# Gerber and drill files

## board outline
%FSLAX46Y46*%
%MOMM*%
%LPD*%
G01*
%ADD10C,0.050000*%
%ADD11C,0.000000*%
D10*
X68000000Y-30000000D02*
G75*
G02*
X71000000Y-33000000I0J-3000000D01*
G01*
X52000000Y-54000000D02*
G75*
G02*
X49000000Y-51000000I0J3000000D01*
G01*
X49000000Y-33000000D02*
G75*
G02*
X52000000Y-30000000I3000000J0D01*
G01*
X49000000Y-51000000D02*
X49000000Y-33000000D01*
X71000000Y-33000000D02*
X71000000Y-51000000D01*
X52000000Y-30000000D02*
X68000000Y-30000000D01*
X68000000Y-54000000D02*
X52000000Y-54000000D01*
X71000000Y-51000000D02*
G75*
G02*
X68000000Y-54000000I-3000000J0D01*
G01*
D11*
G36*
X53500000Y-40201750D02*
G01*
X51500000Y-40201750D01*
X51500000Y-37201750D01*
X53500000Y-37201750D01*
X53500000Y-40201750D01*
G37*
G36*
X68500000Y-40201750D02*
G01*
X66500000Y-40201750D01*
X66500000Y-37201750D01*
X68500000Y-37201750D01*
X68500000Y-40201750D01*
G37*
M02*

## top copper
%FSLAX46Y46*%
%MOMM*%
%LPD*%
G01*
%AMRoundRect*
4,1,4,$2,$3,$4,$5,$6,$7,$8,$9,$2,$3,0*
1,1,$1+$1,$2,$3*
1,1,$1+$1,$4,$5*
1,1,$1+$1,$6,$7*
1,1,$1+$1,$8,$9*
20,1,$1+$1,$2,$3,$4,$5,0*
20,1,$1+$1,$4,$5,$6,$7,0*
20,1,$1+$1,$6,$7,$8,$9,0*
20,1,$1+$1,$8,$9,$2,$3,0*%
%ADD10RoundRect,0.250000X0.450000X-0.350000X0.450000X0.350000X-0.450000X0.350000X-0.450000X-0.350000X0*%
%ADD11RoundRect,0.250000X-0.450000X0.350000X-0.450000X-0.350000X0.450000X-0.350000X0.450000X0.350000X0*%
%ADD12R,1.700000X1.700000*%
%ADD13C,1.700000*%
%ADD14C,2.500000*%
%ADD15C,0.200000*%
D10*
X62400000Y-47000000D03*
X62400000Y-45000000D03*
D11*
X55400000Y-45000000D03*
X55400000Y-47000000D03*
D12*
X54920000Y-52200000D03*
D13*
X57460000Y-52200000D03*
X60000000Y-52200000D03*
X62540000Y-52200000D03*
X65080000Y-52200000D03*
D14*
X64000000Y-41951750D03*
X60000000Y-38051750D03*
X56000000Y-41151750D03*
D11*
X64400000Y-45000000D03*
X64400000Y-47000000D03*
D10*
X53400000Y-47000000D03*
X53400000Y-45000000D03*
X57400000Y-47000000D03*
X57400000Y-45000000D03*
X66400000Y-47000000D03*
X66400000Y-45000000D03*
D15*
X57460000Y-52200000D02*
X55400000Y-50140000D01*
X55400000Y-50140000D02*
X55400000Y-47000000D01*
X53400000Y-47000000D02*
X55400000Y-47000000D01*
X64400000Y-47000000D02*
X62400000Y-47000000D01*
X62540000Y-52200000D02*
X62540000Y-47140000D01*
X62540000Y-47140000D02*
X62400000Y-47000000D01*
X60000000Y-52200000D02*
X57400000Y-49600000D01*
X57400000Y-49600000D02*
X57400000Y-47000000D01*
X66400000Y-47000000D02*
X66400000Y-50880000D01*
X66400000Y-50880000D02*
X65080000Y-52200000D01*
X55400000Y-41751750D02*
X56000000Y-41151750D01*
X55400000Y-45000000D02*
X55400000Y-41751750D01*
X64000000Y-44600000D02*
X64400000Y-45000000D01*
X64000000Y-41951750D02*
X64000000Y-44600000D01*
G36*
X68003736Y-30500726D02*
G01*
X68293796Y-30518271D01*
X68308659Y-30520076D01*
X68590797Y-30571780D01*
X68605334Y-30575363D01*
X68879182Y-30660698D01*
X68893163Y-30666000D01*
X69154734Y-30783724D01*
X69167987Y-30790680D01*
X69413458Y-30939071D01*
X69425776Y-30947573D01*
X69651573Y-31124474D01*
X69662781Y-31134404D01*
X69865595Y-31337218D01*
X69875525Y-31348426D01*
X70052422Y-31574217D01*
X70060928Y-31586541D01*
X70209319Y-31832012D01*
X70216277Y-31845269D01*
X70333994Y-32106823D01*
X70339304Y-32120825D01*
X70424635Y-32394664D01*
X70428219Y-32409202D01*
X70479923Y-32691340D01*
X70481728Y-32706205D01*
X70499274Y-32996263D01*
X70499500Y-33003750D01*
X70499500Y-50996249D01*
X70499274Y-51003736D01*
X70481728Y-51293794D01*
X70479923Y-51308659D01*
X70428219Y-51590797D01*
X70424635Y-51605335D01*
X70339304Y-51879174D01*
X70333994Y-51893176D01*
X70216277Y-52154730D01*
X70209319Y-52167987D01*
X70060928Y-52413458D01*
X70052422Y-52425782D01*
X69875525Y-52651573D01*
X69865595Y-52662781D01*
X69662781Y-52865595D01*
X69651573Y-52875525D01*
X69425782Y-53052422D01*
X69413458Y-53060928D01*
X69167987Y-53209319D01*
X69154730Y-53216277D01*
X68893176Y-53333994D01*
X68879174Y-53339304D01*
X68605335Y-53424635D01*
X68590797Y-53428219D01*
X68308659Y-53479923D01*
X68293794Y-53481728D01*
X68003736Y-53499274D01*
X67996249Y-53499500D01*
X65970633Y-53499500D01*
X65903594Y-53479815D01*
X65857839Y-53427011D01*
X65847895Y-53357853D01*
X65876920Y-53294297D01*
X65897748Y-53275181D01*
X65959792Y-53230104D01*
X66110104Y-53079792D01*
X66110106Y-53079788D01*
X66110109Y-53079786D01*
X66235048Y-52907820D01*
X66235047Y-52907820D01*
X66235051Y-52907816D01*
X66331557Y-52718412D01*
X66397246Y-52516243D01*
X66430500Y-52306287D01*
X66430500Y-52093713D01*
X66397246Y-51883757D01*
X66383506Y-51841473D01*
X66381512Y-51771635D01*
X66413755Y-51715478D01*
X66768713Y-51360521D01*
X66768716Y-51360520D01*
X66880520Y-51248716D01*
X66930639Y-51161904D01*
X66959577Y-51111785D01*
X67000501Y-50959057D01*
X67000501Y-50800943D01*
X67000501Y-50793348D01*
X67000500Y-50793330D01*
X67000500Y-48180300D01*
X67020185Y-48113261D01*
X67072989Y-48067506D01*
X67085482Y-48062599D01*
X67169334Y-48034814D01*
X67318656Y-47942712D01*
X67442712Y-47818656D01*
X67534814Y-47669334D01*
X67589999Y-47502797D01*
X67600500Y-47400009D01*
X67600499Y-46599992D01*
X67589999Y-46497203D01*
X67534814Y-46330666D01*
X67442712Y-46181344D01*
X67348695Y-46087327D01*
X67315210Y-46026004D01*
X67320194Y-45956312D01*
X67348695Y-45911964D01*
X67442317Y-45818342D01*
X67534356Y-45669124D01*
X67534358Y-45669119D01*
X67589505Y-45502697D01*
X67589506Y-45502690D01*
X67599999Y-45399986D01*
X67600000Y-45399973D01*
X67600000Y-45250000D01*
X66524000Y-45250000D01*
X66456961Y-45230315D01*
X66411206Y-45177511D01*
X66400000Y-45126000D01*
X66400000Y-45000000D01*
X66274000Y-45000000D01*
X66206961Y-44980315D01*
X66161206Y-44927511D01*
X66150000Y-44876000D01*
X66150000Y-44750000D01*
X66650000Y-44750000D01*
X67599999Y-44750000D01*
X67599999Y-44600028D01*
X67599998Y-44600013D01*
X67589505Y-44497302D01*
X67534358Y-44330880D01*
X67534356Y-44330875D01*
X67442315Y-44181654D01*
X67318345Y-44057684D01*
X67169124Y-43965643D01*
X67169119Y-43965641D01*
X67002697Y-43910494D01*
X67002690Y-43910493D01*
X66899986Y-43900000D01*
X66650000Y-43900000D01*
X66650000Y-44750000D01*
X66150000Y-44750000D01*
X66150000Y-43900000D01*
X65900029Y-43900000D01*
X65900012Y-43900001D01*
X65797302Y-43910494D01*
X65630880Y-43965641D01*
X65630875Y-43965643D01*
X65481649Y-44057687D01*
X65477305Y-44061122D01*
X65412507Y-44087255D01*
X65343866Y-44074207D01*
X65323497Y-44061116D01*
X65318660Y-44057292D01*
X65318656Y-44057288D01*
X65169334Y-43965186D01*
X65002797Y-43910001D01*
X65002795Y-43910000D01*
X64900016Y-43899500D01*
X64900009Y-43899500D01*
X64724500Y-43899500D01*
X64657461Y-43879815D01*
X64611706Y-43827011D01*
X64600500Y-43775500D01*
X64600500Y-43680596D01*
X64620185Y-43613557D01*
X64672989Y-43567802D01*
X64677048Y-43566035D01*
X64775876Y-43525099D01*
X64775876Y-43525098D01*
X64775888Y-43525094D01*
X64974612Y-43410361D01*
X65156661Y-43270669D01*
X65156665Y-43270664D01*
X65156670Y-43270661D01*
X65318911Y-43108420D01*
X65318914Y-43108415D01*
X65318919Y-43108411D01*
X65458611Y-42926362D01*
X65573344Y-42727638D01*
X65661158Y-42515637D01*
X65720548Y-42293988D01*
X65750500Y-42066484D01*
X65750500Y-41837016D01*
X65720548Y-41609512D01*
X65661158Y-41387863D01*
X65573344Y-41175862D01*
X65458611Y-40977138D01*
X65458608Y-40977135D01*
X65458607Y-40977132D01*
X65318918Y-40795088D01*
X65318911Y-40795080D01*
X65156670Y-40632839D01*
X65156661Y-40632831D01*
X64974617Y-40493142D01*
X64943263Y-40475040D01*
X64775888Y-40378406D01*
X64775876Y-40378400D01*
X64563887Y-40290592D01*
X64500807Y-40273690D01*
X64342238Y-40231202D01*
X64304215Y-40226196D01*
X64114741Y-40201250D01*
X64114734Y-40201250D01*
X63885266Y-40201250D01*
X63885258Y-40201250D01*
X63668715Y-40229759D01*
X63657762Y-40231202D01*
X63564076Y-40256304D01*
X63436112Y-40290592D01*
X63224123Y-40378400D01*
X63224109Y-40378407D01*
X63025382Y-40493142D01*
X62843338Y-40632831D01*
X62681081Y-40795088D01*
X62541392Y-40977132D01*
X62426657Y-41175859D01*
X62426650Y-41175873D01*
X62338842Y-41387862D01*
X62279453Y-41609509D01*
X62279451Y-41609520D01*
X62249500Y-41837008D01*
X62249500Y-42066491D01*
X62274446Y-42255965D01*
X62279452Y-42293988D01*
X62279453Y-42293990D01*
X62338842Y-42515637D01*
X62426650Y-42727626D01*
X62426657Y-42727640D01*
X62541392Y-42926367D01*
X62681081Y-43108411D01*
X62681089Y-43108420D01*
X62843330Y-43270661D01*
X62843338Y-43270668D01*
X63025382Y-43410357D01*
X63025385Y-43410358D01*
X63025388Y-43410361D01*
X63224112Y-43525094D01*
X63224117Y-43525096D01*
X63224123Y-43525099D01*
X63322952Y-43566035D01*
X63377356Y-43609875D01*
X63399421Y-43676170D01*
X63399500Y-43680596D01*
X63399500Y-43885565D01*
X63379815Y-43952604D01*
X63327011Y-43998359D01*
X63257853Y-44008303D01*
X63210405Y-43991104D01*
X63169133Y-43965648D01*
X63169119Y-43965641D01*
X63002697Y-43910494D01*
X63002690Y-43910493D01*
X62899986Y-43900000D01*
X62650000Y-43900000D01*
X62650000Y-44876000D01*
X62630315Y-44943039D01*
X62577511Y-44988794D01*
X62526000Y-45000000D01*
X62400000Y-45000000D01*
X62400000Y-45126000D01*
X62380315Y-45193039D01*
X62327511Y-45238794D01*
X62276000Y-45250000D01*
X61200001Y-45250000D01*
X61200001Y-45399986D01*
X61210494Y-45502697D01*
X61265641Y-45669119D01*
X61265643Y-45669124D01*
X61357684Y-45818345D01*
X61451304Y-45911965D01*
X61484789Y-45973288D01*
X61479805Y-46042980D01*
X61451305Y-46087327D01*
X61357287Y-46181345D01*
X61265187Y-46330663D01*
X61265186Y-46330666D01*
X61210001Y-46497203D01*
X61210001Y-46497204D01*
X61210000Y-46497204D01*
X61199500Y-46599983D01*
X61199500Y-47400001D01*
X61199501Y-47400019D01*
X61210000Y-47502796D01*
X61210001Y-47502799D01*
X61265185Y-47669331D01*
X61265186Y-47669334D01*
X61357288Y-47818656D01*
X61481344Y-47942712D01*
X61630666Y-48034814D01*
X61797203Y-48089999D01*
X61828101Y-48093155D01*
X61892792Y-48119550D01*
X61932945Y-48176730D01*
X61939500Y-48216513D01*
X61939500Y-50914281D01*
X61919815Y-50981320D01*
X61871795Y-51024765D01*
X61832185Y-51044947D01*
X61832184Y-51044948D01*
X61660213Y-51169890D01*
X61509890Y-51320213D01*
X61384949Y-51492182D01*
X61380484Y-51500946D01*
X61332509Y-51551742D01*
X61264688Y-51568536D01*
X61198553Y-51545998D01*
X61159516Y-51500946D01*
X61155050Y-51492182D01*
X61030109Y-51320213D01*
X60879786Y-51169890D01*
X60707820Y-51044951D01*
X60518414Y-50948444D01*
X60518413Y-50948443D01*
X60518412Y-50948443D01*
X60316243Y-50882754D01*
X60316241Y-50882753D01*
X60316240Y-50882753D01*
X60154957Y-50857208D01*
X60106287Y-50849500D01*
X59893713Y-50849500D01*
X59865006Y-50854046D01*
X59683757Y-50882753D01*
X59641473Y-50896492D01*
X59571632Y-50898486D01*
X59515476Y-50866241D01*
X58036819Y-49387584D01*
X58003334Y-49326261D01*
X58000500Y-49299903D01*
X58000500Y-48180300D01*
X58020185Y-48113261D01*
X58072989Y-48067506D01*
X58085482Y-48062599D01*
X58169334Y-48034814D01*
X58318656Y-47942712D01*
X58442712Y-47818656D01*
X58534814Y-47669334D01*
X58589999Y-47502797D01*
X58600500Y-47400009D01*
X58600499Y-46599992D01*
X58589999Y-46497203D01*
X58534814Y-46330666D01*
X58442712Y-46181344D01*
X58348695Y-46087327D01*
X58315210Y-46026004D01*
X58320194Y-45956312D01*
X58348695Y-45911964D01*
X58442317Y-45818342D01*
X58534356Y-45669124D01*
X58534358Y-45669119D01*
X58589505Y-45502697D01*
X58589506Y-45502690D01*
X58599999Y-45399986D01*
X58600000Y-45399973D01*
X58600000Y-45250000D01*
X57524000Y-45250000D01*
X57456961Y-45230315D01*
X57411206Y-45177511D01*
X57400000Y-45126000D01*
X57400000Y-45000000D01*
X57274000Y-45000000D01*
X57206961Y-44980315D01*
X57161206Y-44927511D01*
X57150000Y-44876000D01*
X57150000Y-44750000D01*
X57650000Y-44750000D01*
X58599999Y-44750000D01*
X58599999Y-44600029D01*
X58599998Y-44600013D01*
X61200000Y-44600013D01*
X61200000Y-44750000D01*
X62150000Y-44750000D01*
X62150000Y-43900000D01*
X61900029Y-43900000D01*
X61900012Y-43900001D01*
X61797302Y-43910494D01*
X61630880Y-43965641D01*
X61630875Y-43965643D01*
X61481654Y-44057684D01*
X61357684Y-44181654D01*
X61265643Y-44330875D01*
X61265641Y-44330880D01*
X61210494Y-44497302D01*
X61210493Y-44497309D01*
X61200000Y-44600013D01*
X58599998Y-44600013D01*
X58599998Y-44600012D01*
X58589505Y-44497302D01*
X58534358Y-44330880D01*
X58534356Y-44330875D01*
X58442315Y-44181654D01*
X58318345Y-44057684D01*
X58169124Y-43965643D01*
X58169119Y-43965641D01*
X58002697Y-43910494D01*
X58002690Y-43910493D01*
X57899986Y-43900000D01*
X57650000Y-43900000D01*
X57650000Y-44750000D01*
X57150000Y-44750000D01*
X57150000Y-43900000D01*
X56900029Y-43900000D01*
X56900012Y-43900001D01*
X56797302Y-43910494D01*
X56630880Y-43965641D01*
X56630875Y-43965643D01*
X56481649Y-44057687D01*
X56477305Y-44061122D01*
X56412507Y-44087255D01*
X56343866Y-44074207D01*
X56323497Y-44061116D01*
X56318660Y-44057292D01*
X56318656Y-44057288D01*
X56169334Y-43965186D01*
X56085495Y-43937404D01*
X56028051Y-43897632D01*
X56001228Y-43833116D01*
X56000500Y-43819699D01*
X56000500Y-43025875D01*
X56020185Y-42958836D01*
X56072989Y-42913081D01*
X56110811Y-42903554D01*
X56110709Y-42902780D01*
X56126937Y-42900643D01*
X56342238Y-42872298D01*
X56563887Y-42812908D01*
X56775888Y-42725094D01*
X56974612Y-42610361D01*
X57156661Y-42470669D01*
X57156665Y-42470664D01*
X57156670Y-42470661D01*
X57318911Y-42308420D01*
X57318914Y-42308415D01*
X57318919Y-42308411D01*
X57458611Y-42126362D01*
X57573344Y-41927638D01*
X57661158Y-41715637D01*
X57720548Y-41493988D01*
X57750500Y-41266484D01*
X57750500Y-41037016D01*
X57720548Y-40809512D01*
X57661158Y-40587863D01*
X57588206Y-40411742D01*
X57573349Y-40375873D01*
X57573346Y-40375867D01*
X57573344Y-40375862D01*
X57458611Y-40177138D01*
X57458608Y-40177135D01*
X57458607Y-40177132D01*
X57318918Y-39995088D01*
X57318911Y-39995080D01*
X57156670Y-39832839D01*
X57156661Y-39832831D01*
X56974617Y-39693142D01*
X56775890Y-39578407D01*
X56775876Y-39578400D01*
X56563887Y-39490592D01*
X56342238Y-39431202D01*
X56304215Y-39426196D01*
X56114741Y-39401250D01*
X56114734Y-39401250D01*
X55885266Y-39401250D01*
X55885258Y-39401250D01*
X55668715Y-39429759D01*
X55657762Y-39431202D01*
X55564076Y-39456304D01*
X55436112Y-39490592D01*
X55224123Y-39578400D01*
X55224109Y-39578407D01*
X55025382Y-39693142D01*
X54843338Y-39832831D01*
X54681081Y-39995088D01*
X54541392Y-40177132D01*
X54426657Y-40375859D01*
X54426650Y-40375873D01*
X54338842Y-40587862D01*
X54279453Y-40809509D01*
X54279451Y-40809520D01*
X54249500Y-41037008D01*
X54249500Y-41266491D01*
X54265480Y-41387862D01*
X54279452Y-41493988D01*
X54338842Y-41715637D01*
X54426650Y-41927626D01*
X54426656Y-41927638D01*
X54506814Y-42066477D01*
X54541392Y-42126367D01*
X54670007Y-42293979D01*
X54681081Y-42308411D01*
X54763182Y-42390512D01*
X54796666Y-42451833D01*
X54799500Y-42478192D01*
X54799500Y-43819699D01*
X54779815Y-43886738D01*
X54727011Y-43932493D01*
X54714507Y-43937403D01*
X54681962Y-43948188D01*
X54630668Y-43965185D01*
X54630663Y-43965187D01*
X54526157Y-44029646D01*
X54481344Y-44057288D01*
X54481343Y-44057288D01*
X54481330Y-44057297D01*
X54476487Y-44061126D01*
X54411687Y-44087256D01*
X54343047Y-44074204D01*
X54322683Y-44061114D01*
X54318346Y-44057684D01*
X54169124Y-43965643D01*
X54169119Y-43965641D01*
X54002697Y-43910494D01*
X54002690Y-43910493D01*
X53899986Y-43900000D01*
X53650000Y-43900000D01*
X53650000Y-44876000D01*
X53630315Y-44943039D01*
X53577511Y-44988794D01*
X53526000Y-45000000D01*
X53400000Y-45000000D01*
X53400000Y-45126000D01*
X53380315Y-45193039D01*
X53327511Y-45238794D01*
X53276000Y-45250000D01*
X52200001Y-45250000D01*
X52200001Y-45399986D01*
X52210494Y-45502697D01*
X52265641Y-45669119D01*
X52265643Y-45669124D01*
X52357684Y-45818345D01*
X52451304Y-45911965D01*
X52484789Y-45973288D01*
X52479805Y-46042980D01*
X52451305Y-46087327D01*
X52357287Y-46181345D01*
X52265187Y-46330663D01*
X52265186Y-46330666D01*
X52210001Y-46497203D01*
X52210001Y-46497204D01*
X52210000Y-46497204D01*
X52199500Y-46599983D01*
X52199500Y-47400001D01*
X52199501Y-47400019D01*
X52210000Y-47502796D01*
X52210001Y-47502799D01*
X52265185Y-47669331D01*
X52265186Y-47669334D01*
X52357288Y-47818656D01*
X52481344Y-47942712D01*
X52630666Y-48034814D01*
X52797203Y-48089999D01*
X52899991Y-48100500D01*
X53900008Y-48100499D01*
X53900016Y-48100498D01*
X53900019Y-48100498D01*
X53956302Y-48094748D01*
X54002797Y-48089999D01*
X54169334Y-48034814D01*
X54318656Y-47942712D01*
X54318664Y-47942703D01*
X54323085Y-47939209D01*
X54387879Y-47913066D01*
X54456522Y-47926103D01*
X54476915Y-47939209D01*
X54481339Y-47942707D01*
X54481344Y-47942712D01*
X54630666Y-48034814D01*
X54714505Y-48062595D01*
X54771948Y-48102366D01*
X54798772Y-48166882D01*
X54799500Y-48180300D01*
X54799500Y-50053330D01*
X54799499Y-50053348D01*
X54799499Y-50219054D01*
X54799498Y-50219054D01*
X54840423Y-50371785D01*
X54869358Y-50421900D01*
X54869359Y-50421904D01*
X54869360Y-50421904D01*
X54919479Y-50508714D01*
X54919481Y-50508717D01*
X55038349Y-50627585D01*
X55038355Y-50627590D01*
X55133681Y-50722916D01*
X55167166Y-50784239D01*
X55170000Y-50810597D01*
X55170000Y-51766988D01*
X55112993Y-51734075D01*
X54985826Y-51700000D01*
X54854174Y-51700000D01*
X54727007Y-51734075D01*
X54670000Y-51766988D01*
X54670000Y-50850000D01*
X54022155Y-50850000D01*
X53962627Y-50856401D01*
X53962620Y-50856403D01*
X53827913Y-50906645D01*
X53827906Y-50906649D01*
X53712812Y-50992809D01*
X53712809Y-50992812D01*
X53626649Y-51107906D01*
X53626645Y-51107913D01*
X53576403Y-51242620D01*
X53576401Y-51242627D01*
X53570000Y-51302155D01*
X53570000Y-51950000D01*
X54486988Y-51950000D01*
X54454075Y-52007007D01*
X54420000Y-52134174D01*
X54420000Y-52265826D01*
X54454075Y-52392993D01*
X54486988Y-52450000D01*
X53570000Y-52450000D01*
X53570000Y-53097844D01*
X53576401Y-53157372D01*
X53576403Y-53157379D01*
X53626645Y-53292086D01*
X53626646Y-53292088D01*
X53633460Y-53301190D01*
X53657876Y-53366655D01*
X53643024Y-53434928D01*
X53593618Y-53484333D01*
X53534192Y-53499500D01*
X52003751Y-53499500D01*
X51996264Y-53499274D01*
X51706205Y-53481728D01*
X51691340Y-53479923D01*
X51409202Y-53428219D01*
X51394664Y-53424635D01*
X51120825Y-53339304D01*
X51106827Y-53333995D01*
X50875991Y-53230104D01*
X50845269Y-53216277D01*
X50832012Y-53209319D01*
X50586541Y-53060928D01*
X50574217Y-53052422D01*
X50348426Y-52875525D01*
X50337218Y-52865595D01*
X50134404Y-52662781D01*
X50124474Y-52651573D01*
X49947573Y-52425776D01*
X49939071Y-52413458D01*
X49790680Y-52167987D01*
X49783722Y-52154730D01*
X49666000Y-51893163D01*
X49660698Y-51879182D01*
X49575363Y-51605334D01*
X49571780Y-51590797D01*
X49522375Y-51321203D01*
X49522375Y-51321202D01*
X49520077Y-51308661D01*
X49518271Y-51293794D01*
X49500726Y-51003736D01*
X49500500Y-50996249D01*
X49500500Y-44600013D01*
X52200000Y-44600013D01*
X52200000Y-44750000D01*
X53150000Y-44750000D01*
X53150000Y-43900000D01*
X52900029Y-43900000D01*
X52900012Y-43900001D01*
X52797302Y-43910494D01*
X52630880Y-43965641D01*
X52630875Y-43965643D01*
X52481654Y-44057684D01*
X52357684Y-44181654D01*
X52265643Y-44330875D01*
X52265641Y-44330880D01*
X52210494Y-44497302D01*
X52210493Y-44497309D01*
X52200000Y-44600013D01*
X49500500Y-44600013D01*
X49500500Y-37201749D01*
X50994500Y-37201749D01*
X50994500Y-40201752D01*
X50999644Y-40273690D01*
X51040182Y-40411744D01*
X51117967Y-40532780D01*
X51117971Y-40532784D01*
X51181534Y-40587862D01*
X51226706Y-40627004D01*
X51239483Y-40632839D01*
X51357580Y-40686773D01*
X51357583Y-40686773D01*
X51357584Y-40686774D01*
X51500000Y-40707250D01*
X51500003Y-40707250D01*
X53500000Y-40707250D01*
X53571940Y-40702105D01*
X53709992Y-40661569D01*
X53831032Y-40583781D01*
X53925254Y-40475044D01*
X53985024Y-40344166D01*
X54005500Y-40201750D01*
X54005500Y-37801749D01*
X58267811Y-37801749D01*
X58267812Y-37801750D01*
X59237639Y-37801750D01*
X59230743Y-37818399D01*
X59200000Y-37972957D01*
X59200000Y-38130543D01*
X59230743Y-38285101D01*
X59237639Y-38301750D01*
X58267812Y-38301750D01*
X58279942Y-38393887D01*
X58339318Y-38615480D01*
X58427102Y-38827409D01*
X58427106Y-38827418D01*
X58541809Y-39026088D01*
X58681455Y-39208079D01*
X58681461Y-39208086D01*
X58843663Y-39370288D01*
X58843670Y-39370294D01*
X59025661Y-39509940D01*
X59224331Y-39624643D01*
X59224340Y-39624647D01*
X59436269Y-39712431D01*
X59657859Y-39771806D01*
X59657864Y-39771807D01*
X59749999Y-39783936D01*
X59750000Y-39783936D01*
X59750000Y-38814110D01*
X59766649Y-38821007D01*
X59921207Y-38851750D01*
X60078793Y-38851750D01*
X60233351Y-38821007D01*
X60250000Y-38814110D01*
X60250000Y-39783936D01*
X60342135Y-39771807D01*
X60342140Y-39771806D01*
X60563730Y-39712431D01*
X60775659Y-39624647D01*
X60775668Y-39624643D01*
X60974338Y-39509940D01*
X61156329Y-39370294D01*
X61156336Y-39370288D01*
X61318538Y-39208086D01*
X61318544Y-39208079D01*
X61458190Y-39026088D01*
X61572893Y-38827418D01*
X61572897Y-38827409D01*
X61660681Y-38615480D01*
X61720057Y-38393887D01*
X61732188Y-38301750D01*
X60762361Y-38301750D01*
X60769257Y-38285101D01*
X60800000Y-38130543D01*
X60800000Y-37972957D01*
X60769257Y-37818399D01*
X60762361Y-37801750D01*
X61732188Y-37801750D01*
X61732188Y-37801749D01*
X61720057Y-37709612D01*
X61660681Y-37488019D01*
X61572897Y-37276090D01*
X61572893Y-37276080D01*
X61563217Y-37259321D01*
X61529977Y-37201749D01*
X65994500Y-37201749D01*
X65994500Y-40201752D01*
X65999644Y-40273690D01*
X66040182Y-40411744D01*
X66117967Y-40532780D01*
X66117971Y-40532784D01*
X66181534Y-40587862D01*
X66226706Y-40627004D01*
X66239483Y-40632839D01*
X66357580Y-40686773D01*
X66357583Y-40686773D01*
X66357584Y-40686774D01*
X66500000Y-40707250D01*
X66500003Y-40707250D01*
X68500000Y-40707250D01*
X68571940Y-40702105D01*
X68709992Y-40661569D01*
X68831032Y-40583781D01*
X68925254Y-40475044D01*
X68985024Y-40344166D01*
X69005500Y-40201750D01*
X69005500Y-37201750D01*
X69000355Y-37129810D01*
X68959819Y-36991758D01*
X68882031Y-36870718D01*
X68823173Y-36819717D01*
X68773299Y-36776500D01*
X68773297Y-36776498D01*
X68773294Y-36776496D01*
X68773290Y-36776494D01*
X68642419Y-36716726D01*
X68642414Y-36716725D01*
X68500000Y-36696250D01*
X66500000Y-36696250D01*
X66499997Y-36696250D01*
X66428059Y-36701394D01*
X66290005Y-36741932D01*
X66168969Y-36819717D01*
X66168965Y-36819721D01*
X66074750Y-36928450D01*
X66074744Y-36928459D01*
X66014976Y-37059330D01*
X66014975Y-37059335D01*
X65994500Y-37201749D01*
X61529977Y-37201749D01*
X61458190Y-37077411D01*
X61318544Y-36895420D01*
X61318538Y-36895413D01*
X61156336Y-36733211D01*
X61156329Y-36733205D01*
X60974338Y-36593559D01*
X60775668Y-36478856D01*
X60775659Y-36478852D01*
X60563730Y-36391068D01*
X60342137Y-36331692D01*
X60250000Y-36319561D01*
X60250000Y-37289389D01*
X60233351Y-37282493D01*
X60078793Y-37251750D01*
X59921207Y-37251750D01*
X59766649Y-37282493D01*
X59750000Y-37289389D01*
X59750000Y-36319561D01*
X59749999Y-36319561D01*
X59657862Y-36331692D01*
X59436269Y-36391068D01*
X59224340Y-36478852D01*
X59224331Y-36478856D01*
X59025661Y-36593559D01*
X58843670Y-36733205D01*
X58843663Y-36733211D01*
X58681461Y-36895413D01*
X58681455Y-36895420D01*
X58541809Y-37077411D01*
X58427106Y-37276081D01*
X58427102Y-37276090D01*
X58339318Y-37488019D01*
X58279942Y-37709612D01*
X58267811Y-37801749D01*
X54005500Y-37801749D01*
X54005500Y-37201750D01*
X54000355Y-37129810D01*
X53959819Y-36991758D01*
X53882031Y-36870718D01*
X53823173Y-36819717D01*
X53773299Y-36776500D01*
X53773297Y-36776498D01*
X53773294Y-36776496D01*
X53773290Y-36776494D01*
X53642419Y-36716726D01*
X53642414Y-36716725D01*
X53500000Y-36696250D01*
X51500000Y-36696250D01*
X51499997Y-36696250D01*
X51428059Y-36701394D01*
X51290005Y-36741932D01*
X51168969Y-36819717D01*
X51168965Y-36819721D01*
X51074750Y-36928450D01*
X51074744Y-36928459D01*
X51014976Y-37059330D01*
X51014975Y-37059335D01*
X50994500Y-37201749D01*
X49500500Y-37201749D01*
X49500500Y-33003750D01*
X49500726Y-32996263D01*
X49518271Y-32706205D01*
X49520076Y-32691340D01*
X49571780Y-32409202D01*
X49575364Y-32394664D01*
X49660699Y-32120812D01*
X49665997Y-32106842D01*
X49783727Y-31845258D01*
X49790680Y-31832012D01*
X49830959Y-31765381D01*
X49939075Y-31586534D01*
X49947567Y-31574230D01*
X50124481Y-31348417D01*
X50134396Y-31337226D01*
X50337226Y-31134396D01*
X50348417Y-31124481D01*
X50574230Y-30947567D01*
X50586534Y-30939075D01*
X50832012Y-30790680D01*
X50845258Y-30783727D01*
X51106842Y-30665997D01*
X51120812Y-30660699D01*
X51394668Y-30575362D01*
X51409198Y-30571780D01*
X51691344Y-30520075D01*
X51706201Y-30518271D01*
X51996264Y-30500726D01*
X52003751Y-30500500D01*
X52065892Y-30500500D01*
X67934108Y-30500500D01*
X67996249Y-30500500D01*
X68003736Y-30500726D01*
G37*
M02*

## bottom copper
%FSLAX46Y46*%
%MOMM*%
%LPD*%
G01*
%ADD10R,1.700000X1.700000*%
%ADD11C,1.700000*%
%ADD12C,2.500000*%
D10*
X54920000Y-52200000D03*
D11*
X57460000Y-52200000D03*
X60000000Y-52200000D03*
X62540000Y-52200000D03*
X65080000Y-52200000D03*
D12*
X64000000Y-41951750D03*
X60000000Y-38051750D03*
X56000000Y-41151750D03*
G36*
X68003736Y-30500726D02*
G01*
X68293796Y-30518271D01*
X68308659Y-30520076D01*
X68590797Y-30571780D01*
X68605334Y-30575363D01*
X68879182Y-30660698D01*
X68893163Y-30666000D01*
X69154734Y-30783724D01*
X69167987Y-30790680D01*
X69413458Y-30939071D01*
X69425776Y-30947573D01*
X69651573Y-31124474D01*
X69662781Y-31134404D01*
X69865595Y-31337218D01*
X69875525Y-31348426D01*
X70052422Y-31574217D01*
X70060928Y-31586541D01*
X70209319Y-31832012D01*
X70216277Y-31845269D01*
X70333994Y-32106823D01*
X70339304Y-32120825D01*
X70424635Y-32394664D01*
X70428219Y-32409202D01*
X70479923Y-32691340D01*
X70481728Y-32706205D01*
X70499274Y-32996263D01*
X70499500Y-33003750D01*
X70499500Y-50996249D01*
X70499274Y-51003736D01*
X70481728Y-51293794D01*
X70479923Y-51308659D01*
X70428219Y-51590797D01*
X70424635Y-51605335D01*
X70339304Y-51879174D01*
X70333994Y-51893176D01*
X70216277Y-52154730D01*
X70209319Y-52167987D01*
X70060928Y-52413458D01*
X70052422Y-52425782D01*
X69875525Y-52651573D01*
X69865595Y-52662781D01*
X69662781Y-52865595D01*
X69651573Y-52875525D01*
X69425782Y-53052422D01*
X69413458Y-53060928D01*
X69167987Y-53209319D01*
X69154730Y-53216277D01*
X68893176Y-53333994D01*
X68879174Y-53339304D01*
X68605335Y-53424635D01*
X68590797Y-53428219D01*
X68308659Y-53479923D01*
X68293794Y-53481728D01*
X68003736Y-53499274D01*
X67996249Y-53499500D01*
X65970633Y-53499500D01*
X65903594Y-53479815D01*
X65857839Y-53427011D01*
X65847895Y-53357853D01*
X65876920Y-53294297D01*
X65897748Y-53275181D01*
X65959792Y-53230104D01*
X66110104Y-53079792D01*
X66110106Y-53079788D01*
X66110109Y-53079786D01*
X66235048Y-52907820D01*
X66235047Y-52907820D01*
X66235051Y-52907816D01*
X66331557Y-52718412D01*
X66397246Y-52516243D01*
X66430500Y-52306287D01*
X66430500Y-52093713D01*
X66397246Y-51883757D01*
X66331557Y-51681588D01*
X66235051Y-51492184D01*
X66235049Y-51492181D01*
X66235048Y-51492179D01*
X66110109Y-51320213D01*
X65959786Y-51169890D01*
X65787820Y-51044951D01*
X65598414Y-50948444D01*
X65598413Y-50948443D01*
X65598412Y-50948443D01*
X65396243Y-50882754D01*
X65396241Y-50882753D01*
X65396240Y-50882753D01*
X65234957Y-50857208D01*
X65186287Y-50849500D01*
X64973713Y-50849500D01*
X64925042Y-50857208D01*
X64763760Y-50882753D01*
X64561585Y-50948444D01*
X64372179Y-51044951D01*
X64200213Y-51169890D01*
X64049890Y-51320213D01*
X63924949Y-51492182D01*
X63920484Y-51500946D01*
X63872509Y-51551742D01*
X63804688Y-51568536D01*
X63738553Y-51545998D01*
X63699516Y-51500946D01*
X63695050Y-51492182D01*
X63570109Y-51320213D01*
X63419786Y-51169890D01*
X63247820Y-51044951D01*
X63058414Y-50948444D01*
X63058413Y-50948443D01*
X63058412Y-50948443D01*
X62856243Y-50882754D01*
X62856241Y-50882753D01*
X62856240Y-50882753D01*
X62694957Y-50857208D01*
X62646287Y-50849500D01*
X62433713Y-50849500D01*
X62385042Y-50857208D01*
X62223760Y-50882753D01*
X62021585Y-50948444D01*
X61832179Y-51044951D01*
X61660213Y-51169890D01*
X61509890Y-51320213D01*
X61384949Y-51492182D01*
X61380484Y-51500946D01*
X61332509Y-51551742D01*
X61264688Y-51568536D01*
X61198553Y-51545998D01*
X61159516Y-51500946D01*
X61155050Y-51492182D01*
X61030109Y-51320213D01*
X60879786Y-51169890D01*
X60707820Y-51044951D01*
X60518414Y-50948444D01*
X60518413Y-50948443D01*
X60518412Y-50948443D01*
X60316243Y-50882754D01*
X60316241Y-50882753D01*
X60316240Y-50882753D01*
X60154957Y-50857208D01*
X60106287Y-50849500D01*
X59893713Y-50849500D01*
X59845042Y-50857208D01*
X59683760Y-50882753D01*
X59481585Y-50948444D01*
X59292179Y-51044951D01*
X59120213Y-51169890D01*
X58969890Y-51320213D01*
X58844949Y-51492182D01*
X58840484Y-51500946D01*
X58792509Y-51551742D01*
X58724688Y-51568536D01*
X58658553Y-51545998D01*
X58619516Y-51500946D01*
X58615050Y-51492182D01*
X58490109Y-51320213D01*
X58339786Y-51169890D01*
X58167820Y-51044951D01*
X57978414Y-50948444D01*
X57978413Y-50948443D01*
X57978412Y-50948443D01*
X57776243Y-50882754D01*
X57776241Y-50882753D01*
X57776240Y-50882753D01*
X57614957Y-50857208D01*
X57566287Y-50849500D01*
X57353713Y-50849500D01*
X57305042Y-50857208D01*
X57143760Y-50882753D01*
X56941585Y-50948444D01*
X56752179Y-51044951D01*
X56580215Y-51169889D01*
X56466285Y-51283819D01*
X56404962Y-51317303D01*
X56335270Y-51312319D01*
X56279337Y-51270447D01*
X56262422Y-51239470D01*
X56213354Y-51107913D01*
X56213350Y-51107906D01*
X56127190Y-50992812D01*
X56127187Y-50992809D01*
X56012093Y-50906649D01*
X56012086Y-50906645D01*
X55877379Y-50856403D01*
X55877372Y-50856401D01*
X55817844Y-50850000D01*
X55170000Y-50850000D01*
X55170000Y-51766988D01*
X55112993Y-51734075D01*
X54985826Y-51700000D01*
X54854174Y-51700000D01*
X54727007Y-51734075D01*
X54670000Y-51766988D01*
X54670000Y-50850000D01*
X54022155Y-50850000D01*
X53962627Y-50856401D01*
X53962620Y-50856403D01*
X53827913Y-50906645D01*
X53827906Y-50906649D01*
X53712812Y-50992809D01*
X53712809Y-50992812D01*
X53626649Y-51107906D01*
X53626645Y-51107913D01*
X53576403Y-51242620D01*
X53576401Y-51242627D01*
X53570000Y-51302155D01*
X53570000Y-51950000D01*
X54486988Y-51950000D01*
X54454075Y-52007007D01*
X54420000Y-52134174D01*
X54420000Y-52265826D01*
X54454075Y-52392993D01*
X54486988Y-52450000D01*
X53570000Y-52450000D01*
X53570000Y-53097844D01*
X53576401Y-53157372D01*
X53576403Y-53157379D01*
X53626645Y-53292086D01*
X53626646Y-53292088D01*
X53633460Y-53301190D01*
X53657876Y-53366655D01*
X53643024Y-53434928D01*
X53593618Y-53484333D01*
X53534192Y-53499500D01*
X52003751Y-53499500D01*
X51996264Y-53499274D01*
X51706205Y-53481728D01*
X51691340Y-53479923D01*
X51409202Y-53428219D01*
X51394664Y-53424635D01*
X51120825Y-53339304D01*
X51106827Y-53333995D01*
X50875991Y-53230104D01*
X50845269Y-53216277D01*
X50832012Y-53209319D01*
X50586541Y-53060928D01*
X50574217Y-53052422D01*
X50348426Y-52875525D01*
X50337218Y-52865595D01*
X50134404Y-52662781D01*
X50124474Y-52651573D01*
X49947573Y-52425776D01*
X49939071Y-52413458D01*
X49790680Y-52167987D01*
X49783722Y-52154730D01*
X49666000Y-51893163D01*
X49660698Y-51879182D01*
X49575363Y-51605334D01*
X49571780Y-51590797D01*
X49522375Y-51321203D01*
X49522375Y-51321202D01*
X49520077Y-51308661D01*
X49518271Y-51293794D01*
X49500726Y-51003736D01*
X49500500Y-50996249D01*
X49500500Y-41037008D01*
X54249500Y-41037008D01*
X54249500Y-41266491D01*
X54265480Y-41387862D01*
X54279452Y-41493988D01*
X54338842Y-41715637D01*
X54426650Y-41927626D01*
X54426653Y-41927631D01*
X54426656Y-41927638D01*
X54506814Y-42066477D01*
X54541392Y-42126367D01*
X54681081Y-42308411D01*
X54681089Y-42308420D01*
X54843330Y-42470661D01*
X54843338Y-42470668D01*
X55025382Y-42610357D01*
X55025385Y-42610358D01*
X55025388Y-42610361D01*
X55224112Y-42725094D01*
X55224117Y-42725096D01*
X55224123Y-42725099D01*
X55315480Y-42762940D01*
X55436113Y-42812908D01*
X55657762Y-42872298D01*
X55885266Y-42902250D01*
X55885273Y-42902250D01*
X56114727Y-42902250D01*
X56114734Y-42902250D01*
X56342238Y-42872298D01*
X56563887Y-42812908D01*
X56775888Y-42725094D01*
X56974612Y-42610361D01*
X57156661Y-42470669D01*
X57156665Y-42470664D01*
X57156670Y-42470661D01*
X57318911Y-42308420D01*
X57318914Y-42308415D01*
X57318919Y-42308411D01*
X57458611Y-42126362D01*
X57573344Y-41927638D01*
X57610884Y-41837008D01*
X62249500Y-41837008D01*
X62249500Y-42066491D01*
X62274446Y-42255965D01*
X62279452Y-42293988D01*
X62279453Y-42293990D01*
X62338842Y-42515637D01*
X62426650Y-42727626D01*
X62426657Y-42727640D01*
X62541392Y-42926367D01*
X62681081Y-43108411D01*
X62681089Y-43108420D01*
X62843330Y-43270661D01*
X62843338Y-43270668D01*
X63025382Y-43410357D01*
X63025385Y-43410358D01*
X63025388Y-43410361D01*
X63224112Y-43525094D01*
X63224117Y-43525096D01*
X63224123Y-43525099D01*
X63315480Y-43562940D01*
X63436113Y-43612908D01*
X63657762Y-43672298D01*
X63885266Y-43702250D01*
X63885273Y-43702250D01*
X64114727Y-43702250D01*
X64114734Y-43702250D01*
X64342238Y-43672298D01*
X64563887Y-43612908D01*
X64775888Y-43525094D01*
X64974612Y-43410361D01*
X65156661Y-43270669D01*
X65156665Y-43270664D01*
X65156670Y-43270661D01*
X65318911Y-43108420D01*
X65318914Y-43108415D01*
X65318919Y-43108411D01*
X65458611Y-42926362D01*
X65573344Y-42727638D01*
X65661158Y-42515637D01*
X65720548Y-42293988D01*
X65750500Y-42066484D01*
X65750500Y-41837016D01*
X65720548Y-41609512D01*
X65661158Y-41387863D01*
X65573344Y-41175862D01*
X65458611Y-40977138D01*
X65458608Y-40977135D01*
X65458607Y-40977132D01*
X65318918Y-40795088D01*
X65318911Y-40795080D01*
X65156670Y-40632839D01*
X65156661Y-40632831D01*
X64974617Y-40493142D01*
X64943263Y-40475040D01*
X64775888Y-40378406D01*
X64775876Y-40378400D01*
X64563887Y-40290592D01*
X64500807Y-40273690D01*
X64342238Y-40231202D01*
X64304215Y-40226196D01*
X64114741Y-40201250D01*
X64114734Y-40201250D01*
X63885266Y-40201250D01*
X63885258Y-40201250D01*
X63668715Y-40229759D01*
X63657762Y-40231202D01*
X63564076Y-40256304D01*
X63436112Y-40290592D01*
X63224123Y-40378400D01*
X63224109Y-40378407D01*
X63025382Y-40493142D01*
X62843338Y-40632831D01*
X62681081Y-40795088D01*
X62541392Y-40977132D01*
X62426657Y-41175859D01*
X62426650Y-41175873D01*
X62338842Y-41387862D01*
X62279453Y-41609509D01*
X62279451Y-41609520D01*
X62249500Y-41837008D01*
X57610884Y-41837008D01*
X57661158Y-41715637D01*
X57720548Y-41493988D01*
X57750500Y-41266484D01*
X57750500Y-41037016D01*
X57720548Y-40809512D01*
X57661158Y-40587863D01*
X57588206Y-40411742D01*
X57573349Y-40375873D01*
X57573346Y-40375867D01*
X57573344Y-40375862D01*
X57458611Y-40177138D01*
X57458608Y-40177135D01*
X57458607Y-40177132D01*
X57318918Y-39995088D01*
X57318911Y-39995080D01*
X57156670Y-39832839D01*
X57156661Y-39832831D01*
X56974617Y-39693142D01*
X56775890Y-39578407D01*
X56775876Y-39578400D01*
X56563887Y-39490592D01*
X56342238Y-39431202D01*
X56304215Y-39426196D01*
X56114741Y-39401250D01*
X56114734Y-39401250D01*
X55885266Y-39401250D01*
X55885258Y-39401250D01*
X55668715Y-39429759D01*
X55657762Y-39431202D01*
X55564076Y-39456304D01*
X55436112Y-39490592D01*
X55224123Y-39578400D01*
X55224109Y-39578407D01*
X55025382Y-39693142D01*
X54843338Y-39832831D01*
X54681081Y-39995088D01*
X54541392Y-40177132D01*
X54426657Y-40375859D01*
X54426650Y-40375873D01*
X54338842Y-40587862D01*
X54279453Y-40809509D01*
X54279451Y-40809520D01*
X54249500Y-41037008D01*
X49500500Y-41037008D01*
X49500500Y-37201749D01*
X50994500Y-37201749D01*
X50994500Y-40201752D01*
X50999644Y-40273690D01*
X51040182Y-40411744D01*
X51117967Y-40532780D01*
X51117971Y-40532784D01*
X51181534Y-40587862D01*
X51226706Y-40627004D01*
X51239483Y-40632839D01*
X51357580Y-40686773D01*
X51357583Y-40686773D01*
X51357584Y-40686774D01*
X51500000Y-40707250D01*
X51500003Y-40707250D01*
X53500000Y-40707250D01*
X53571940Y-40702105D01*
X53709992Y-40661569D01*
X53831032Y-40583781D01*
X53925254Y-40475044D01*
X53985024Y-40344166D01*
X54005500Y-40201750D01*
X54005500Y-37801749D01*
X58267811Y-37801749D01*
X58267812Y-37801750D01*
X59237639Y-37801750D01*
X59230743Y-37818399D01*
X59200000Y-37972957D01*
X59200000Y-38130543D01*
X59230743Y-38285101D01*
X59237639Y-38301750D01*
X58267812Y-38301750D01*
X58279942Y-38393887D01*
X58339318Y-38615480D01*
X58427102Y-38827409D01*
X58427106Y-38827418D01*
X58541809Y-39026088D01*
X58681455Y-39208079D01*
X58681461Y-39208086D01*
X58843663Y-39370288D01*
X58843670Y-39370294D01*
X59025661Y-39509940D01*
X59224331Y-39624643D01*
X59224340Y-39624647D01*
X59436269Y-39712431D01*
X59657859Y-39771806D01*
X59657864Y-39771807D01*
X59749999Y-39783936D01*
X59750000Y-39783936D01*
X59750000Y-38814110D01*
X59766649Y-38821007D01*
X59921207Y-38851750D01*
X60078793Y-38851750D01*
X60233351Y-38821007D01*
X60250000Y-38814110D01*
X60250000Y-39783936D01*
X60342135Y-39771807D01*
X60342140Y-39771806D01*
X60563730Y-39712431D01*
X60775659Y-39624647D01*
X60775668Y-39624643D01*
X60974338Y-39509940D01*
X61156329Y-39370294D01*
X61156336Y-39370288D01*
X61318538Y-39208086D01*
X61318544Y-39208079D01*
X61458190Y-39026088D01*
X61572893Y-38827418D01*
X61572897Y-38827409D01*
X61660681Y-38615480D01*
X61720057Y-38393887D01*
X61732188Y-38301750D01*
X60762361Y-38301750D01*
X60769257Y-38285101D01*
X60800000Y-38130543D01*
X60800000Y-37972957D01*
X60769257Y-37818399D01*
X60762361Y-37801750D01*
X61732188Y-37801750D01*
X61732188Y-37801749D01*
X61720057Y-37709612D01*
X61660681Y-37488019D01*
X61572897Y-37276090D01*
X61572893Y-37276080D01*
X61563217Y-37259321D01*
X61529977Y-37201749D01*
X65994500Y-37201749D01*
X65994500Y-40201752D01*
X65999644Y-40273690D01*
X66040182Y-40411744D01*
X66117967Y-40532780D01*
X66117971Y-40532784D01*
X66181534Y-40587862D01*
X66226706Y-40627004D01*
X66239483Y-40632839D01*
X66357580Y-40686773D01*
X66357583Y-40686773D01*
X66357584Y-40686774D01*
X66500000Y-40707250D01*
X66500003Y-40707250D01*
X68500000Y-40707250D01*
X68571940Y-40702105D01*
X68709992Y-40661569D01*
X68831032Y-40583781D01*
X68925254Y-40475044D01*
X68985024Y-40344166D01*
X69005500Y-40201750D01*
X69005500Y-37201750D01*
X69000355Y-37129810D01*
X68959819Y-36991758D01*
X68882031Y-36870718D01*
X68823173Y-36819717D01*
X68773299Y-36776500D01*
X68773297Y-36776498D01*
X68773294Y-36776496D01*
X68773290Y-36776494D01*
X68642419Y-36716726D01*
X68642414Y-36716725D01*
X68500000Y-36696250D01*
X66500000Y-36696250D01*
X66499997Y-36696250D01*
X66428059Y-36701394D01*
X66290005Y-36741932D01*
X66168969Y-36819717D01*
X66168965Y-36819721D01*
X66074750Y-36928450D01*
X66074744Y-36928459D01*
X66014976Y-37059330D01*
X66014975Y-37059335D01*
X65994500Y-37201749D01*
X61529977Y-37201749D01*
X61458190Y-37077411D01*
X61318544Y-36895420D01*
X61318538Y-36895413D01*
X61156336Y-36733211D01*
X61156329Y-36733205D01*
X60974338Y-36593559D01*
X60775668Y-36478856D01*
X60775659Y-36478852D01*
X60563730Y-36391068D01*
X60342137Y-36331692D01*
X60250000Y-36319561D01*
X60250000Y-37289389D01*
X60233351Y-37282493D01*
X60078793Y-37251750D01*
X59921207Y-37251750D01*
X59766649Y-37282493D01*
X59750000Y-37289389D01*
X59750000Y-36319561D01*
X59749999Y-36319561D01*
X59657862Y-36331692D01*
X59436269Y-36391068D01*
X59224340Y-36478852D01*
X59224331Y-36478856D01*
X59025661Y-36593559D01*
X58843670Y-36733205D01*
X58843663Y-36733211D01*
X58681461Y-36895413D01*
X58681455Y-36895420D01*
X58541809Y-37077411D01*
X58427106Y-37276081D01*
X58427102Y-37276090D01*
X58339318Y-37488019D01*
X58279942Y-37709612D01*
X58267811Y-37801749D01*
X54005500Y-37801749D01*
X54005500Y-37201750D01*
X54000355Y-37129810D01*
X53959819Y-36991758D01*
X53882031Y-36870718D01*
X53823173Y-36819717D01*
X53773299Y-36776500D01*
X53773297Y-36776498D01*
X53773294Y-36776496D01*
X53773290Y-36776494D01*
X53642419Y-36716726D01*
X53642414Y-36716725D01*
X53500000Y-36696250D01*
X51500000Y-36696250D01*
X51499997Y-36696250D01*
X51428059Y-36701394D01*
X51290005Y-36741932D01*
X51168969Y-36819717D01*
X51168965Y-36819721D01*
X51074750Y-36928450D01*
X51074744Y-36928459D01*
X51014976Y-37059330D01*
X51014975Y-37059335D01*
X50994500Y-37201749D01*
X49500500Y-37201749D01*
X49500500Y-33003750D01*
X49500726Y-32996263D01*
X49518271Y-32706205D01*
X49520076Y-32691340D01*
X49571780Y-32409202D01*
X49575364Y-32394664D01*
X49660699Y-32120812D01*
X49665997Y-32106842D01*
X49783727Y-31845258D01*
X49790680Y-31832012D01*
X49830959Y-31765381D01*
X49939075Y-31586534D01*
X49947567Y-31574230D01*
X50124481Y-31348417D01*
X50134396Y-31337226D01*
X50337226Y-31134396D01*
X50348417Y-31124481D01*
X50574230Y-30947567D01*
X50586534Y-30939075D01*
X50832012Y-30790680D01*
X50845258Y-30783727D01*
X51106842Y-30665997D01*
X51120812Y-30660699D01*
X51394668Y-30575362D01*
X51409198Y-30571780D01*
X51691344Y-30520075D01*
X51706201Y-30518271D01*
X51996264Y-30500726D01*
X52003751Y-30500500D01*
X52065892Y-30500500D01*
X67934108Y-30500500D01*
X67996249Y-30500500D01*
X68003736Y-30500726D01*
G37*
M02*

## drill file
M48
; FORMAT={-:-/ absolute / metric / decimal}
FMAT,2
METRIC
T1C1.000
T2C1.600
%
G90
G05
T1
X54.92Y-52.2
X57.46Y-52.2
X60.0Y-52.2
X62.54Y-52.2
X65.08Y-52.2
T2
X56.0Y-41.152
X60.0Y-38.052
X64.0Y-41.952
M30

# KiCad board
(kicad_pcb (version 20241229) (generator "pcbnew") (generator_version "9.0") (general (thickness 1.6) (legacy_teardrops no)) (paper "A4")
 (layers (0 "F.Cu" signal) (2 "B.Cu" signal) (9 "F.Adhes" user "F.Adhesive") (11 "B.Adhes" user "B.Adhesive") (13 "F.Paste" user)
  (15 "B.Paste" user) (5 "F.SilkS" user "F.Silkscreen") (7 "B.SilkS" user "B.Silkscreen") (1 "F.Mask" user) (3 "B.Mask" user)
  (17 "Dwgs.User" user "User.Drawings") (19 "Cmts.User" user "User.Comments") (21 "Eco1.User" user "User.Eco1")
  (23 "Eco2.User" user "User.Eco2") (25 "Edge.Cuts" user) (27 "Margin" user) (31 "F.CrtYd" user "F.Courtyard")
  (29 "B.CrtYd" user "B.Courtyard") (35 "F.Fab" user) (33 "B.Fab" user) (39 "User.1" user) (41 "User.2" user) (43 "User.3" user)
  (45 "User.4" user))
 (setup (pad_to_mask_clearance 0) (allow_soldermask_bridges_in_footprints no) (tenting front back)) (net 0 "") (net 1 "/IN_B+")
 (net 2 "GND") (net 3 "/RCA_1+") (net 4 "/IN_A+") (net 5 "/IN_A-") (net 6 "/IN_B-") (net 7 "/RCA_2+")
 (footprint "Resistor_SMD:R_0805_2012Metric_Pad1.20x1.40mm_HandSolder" (layer "F.Cu") (at 62.4 46 90)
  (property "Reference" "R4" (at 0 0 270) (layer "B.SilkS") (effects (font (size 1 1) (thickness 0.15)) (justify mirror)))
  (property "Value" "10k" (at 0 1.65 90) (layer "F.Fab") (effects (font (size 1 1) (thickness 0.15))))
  (pad "1" smd roundrect (at -1 0 90) (size 1.2 1.4) (layers "F.Cu" "F.Mask" "F.Paste") (roundrect_rratio 0.208333) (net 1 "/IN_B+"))
  (pad "2" smd roundrect (at 1 0 90) (size 1.2 1.4) (layers "F.Cu" "F.Mask" "F.Paste") (roundrect_rratio 0.208333) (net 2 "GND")))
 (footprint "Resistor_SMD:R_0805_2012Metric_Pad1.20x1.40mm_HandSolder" (layer "F.Cu") (at 55.4 46 -90)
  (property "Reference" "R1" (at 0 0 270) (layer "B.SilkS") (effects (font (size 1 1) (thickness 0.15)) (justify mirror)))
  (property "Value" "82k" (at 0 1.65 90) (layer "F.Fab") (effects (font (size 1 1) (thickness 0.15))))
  (pad "1" smd roundrect (at -1 0 270) (size 1.2 1.4) (layers "F.Cu" "F.Mask" "F.Paste") (roundrect_rratio 0.208333) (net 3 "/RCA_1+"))
  (pad "2" smd roundrect (at 1 0 270) (size 1.2 1.4) (layers "F.Cu" "F.Mask" "F.Paste") (roundrect_rratio 0.208333) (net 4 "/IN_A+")))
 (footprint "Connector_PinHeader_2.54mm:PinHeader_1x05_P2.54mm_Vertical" (layer "F.Cu") (at 54.92 52.2 90)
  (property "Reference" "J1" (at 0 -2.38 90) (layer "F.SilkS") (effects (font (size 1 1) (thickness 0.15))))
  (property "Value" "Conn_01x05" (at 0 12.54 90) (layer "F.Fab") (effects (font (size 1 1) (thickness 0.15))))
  (pad "1" thru_hole rect (at 0 0 90) (size 1.7 1.7) (drill 1) (layers "*.Cu" "*.Mask") (remove_unused_layers no) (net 2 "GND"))
  (pad "2" thru_hole circle (at 0 2.54 90) (size 1.7 1.7) (drill 1) (layers "*.Cu" "*.Mask") (remove_unused_layers no) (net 4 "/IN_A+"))
  (pad "3" thru_hole circle (at 0 5.08 90) (size 1.7 1.7) (drill 1) (layers "*.Cu" "*.Mask") (remove_unused_layers no) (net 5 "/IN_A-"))
  (pad "4" thru_hole circle (at 0 7.62 90) (size 1.7 1.7) (drill 1) (layers "*.Cu" "*.Mask") (remove_unused_layers no) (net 1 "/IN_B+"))
  (pad "5" thru_hole circle (at 0 10.16 90) (size 1.7 1.7) (drill 1) (layers "*.Cu" "*.Mask") (remove_unused_layers no) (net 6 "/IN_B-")))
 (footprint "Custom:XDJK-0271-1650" (layer "F.Cu") (at 60 40.00175 180)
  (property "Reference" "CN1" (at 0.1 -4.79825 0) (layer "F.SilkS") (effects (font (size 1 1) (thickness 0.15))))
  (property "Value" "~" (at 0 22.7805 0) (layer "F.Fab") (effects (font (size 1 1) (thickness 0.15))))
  (fp_poly (pts (xy 6.5 2.8) (xy 6.5 -0.2) (xy 8.5 -0.2) (xy 8.5 2.8)) (stroke (width 0) (type default)) (fill yes) (layer "Edge.Cuts"))
  (fp_poly (pts (xy -8.5 2.8) (xy -8.5 -0.2) (xy -6.5 -0.2) (xy -6.5 2.8)) (stroke (width 0) (type default)) (fill yes) (layer "Edge.Cuts"))
  (pad "1" thru_hole circle (at -4 -1.95 180) (size 2.5 2.5) (drill 1.6) (layers "*.Cu" "*.Mask") (remove_unused_layers no)
   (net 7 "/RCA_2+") (thermal_bridge_angle 90))
  (pad "2" thru_hole circle (at 0 1.95 180) (size 2.5 2.5) (drill 1.6) (layers "*.Cu" "*.Mask") (remove_unused_layers no) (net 2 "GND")
   (thermal_bridge_angle 90))
  (pad "3" thru_hole circle (at 4 -1.15 180) (size 2.5 2.5) (drill 1.6) (layers "*.Cu" "*.Mask") (remove_unused_layers no) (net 3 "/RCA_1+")
   (thermal_bridge_angle 90)))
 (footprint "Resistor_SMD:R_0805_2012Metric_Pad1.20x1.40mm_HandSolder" (layer "F.Cu") (at 64.4 46 -90)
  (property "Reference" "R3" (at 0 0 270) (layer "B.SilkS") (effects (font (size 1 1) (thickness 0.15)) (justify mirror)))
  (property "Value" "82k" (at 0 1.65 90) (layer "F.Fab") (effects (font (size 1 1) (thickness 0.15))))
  (pad "1" smd roundrect (at -1 0 270) (size 1.2 1.4) (layers "F.Cu" "F.Mask" "F.Paste") (roundrect_rratio 0.208333) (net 7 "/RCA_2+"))
  (pad "2" smd roundrect (at 1 0 270) (size 1.2 1.4) (layers "F.Cu" "F.Mask" "F.Paste") (roundrect_rratio 0.208333) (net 1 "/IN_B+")))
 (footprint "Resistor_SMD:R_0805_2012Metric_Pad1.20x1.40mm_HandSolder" (layer "F.Cu") (at 53.4 46 90)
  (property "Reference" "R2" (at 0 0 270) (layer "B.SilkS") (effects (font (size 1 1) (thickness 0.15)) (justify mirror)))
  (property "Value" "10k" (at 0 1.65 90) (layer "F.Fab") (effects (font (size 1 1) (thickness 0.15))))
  (pad "1" smd roundrect (at -1 0 90) (size 1.2 1.4) (layers "F.Cu" "F.Mask" "F.Paste") (roundrect_rratio 0.208333) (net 4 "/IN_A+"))
  (pad "2" smd roundrect (at 1 0 90) (size 1.2 1.4) (layers "F.Cu" "F.Mask" "F.Paste") (roundrect_rratio 0.208333) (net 2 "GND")))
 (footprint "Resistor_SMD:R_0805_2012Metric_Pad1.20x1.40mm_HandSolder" (layer "F.Cu") (at 57.4 46 90)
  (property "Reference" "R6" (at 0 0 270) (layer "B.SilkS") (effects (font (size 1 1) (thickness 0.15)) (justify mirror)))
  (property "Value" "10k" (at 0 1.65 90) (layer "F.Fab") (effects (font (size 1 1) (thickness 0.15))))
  (pad "1" smd roundrect (at -1 0 90) (size 1.2 1.4) (layers "F.Cu" "F.Mask" "F.Paste") (roundrect_rratio 0.208333) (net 5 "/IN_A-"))
  (pad "2" smd roundrect (at 1 0 90) (size 1.2 1.4) (layers "F.Cu" "F.Mask" "F.Paste") (roundrect_rratio 0.208333) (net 2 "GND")))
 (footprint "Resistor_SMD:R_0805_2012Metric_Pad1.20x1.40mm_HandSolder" (layer "F.Cu") (at 66.4 46 90)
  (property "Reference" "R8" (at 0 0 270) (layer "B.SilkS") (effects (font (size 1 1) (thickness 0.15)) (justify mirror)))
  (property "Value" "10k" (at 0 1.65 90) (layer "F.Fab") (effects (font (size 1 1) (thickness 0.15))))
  (pad "1" smd roundrect (at -1 0 90) (size 1.2 1.4) (layers "F.Cu" "F.Mask" "F.Paste") (roundrect_rratio 0.208333) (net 6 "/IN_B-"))
  (pad "2" smd roundrect (at 1 0 90) (size 1.2 1.4) (layers "F.Cu" "F.Mask" "F.Paste") (roundrect_rratio 0.208333) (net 2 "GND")))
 (gr_arc (start 68 30) (mid 70.12132 30.87868) (end 71 33) (stroke (width 0.05) (type default)) (layer "Edge.Cuts"))
 (gr_arc (start 52 54) (mid 49.87868 53.12132) (end 49 51) (stroke (width 0.05) (type default)) (layer "Edge.Cuts"))
 (gr_arc (start 49 33) (mid 49.87868 30.87868) (end 52 30) (stroke (width 0.05) (type default)) (layer "Edge.Cuts"))
 (gr_line (start 49 51) (end 49 33) (stroke (width 0.05) (type default)) (layer "Edge.Cuts"))
 (gr_line (start 71 33) (end 71 51) (stroke (width 0.05) (type default)) (layer "Edge.Cuts"))
 (gr_line (start 52 30) (end 68 30) (stroke (width 0.05) (type default)) (layer "Edge.Cuts"))
 (gr_line (start 68 54) (end 52 54) (stroke (width 0.05) (type default)) (layer "Edge.Cuts"))
 (gr_arc (start 71 51) (mid 70.12132 53.12132) (end 68 54) (stroke (width 0.05) (type default)) (layer "Edge.Cuts"))
 (segment (start 57.46 52.2) (end 55.4 50.14) (width 0.2) (layer "F.Cu") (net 4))
 (segment (start 55.4 50.14) (end 55.4 47) (width 0.2) (layer "F.Cu") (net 4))
 (segment (start 53.4 47) (end 55.4 47) (width 0.2) (layer "F.Cu") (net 4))
 (segment (start 64.4 47) (end 62.4 47) (width 0.2) (layer "F.Cu") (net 1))
 (segment (start 62.54 52.2) (end 62.54 47.14) (width 0.2) (layer "F.Cu") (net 1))
 (segment (start 62.54 47.14) (end 62.4 47) (width 0.2) (layer "F.Cu") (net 1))
 (segment (start 60 52.2) (end 57.4 49.6) (width 0.2) (layer "F.Cu") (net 5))
 (segment (start 57.4 49.6) (end 57.4 47) (width 0.2) (layer "F.Cu") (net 5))
 (segment (start 66.4 47) (end 66.4 50.88) (width 0.2) (layer "F.Cu") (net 6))
 (segment (start 66.4 50.88) (end 65.08 52.2) (width 0.2) (layer "F.Cu") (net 6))
 (segment (start 55.4 41.75175) (end 56 41.15175) (width 0.2) (layer "F.Cu") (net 3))
 (segment (start 55.4 45) (end 55.4 41.75175) (width 0.2) (layer "F.Cu") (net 3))
 (segment (start 64 44.6) (end 64.4 45) (width 0.2) (layer "F.Cu") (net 7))
 (segment (start 64 41.95175) (end 64 44.6) (width 0.2) (layer "F.Cu") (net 7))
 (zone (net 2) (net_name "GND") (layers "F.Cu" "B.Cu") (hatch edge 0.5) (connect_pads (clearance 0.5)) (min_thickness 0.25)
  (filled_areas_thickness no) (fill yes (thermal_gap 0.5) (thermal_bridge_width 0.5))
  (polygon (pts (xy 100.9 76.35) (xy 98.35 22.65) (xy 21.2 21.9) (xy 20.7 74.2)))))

